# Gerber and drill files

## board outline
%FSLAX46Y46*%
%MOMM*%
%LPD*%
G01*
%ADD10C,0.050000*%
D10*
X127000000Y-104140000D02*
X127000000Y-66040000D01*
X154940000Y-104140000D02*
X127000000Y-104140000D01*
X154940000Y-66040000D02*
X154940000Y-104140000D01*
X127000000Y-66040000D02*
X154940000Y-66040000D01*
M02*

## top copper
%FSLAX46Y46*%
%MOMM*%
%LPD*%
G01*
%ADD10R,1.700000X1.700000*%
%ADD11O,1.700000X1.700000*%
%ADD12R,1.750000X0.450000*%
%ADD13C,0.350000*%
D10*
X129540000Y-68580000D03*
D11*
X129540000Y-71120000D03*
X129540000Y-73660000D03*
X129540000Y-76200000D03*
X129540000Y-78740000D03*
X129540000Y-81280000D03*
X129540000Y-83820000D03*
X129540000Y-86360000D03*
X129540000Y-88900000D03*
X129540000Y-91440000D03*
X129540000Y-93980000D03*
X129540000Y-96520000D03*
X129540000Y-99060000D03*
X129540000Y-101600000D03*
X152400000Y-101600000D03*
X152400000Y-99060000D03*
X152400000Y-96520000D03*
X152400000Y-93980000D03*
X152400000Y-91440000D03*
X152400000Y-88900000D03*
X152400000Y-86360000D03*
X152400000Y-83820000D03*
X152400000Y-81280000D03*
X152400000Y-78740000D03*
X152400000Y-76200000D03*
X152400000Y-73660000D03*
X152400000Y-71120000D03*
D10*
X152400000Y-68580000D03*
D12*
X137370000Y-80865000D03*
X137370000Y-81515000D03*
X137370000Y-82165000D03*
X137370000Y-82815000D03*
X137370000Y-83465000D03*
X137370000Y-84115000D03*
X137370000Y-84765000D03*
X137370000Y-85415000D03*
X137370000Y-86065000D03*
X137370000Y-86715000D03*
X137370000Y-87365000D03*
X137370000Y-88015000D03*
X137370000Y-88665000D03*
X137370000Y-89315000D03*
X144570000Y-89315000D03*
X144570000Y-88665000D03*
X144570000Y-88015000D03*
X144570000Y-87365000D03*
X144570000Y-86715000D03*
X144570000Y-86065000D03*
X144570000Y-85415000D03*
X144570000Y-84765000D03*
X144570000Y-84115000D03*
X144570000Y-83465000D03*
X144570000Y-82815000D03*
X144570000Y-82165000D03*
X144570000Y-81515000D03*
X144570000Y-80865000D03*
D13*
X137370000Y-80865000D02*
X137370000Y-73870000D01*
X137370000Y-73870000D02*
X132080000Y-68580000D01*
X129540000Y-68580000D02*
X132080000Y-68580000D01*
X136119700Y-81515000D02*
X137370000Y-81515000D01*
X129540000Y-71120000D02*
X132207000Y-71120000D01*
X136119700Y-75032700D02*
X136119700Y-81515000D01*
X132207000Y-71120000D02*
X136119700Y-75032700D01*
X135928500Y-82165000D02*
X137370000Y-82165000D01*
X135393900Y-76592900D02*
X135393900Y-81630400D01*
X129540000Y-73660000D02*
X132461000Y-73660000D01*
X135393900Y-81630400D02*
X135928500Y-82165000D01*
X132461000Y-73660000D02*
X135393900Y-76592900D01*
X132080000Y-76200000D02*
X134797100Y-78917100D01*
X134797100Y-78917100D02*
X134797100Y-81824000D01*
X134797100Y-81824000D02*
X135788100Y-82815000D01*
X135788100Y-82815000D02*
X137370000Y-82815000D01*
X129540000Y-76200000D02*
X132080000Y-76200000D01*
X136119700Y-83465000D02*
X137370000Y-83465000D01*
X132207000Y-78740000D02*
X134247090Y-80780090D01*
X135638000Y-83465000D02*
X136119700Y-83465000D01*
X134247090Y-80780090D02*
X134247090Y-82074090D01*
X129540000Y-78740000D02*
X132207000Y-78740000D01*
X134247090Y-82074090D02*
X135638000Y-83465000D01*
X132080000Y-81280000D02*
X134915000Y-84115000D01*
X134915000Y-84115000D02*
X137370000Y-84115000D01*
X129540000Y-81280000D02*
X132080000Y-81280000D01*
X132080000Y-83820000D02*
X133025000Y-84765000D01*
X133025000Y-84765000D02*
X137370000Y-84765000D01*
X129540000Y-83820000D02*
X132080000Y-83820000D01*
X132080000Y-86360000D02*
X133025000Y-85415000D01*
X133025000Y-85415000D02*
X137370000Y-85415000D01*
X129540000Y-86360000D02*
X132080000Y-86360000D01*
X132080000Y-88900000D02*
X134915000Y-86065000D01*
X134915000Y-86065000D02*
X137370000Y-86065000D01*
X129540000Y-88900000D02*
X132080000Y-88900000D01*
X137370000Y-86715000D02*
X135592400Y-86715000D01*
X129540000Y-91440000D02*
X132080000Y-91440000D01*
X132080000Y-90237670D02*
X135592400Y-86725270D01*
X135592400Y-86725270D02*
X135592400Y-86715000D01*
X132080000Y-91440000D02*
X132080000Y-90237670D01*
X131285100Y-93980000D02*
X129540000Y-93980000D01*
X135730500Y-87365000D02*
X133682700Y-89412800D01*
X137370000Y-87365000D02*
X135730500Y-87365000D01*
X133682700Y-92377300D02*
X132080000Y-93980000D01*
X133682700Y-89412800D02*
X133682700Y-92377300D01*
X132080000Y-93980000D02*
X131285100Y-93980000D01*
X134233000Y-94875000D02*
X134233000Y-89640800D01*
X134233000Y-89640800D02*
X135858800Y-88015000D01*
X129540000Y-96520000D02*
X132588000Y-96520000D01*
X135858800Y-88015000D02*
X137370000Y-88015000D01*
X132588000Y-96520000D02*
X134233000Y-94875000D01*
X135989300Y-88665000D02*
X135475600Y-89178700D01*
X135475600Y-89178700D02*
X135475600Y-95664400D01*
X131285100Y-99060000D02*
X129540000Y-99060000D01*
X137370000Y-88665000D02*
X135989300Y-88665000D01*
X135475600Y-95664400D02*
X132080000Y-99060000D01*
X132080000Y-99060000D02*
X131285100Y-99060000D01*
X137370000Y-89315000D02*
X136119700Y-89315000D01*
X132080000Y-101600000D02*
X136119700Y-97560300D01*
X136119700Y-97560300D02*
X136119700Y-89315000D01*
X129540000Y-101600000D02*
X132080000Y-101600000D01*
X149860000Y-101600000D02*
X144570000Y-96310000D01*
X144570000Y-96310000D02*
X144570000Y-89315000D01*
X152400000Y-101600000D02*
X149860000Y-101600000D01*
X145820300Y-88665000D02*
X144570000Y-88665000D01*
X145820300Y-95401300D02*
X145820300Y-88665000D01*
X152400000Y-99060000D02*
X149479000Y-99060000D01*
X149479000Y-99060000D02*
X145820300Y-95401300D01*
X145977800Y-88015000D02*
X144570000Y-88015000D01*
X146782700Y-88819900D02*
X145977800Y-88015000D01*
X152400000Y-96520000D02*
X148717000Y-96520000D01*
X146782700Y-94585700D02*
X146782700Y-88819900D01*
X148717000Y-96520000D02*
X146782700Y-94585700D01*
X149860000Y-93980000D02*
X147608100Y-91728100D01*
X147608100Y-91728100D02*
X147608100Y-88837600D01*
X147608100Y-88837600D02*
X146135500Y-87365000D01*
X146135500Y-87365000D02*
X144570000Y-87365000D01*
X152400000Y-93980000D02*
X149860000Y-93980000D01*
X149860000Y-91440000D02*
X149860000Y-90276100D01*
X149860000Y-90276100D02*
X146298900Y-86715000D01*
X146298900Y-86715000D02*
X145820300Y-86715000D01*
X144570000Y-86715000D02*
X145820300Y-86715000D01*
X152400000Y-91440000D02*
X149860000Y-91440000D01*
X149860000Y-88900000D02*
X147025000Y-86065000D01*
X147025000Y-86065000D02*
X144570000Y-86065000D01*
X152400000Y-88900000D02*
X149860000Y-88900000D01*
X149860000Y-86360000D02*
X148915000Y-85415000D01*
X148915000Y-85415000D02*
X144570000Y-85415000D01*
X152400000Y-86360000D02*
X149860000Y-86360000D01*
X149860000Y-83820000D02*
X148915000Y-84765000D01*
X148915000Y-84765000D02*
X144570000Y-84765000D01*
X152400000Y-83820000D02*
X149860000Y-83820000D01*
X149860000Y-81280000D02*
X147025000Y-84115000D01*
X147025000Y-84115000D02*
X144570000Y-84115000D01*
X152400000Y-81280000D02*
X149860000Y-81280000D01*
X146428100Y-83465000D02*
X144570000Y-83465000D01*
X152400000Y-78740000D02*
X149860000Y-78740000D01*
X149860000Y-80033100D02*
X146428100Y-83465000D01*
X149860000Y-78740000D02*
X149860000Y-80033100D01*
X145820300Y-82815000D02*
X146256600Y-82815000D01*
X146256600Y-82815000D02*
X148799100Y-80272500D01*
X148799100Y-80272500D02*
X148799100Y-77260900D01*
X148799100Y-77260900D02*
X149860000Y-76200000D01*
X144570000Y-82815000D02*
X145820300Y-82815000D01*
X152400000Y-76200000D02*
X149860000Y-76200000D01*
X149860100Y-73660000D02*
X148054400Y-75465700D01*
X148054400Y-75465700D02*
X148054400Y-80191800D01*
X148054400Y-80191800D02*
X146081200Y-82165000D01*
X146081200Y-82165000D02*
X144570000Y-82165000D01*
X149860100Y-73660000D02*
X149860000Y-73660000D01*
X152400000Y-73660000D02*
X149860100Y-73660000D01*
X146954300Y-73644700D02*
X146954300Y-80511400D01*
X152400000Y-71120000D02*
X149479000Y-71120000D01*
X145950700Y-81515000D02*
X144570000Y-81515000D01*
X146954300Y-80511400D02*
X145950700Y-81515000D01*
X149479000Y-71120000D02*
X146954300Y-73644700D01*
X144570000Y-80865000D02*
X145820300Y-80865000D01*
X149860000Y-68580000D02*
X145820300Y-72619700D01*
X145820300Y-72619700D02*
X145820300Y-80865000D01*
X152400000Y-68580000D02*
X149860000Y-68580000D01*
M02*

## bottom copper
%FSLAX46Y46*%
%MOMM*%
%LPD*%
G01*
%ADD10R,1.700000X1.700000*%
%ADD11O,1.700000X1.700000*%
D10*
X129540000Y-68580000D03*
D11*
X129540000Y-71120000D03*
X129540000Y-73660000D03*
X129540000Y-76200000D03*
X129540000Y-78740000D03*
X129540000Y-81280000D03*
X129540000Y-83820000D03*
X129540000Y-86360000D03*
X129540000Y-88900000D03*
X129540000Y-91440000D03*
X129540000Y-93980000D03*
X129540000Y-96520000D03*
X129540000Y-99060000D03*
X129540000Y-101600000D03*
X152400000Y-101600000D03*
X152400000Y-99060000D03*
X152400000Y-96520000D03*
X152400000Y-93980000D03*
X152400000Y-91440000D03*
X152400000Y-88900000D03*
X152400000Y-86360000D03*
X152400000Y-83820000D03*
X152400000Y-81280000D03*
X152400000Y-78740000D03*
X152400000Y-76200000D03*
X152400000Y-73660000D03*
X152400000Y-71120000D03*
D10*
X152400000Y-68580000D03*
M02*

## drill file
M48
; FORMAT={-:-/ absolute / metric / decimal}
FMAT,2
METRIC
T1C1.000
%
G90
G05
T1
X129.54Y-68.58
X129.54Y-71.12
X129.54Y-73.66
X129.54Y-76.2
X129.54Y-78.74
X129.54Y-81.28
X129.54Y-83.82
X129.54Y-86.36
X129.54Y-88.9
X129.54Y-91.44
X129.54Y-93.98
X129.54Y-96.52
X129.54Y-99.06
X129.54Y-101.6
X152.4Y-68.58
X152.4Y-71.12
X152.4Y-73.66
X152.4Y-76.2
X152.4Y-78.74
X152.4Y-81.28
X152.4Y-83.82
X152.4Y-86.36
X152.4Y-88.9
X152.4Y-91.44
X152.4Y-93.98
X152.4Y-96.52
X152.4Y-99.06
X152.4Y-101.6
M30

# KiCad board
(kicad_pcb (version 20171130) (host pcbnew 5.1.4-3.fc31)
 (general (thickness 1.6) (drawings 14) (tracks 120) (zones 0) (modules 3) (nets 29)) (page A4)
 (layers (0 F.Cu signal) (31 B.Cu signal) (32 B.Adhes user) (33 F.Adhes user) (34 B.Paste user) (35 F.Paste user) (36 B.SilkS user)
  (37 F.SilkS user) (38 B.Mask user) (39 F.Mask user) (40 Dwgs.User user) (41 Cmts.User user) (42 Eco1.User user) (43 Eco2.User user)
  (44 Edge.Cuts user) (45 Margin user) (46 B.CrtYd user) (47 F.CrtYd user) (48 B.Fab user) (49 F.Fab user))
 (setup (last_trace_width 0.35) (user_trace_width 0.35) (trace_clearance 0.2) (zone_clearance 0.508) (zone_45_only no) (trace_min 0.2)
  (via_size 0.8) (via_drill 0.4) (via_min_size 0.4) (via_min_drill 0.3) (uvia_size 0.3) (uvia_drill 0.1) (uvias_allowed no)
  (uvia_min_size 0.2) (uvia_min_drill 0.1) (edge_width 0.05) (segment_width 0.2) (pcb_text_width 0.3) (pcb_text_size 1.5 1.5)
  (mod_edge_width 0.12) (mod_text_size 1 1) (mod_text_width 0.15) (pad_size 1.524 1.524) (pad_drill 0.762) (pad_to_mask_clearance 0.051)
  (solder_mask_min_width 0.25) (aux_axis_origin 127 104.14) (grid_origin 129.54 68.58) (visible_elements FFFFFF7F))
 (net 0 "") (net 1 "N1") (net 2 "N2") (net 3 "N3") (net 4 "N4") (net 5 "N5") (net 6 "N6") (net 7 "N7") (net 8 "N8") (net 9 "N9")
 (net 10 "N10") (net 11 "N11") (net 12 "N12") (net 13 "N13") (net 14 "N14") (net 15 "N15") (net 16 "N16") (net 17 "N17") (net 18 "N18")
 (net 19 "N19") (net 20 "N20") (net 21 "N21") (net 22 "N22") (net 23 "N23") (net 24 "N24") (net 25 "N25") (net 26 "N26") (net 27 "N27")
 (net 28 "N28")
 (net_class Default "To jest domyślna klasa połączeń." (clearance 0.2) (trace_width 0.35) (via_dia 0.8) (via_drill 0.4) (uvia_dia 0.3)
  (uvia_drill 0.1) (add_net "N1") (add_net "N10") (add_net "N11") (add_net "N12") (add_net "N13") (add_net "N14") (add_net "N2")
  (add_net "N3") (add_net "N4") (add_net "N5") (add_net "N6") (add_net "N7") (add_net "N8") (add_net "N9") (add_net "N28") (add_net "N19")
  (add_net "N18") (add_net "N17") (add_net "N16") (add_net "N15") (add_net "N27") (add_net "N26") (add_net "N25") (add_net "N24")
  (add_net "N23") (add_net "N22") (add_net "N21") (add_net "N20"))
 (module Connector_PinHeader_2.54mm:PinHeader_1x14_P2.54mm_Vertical (layer B.Cu) (at 129.54 68.58 180)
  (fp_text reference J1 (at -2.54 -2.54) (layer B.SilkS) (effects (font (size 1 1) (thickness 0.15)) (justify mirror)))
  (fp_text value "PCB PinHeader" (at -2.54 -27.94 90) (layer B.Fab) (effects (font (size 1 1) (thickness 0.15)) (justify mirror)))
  (pad 1 thru_hole rect (at 0 0 180) (size 1.7 1.7) (drill 1) (layers *.Cu *.Mask) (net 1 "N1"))
  (pad 2 thru_hole oval (at 0 -2.54 180) (size 1.7 1.7) (drill 1) (layers *.Cu *.Mask) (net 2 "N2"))
  (pad 3 thru_hole oval (at 0 -5.08 180) (size 1.7 1.7) (drill 1) (layers *.Cu *.Mask) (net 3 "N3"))
  (pad 4 thru_hole oval (at 0 -7.62 180) (size 1.7 1.7) (drill 1) (layers *.Cu *.Mask) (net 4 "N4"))
  (pad 5 thru_hole oval (at 0 -10.16 180) (size 1.7 1.7) (drill 1) (layers *.Cu *.Mask) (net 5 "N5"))
  (pad 6 thru_hole oval (at 0 -12.7 180) (size 1.7 1.7) (drill 1) (layers *.Cu *.Mask) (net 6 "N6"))
  (pad 7 thru_hole oval (at 0 -15.24 180) (size 1.7 1.7) (drill 1) (layers *.Cu *.Mask) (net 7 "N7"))
  (pad 8 thru_hole oval (at 0 -17.78 180) (size 1.7 1.7) (drill 1) (layers *.Cu *.Mask) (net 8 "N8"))
  (pad 9 thru_hole oval (at 0 -20.32 180) (size 1.7 1.7) (drill 1) (layers *.Cu *.Mask) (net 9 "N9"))
  (pad 10 thru_hole oval (at 0 -22.86 180) (size 1.7 1.7) (drill 1) (layers *.Cu *.Mask) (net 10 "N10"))
  (pad 11 thru_hole oval (at 0 -25.4 180) (size 1.7 1.7) (drill 1) (layers *.Cu *.Mask) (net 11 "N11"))
  (pad 12 thru_hole oval (at 0 -27.94 180) (size 1.7 1.7) (drill 1) (layers *.Cu *.Mask) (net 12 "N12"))
  (pad 13 thru_hole oval (at 0 -30.48 180) (size 1.7 1.7) (drill 1) (layers *.Cu *.Mask) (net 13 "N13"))
  (pad 14 thru_hole oval (at 0 -33.02 180) (size 1.7 1.7) (drill 1) (layers *.Cu *.Mask) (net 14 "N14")))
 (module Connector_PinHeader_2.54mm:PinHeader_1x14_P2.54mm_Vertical (layer B.Cu) (at 152.4 68.58 180)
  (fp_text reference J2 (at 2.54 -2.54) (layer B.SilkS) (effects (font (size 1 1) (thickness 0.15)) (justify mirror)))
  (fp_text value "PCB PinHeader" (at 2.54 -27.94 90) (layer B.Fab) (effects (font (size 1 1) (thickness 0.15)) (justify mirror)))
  (pad 14 thru_hole oval (at 0 -33.02 180) (size 1.7 1.7) (drill 1) (layers *.Cu *.Mask) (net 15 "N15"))
  (pad 13 thru_hole oval (at 0 -30.48 180) (size 1.7 1.7) (drill 1) (layers *.Cu *.Mask) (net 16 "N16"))
  (pad 12 thru_hole oval (at 0 -27.94 180) (size 1.7 1.7) (drill 1) (layers *.Cu *.Mask) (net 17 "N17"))
  (pad 11 thru_hole oval (at 0 -25.4 180) (size 1.7 1.7) (drill 1) (layers *.Cu *.Mask) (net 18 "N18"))
  (pad 10 thru_hole oval (at 0 -22.86 180) (size 1.7 1.7) (drill 1) (layers *.Cu *.Mask) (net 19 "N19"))
  (pad 9 thru_hole oval (at 0 -20.32 180) (size 1.7 1.7) (drill 1) (layers *.Cu *.Mask) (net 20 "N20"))
  (pad 8 thru_hole oval (at 0 -17.78 180) (size 1.7 1.7) (drill 1) (layers *.Cu *.Mask) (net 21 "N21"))
  (pad 7 thru_hole oval (at 0 -15.24 180) (size 1.7 1.7) (drill 1) (layers *.Cu *.Mask) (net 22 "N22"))
  (pad 6 thru_hole oval (at 0 -12.7 180) (size 1.7 1.7) (drill 1) (layers *.Cu *.Mask) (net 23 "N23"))
  (pad 5 thru_hole oval (at 0 -10.16 180) (size 1.7 1.7) (drill 1) (layers *.Cu *.Mask) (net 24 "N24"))
  (pad 4 thru_hole oval (at 0 -7.62 180) (size 1.7 1.7) (drill 1) (layers *.Cu *.Mask) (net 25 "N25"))
  (pad 3 thru_hole oval (at 0 -5.08 180) (size 1.7 1.7) (drill 1) (layers *.Cu *.Mask) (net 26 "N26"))
  (pad 2 thru_hole oval (at 0 -2.54 180) (size 1.7 1.7) (drill 1) (layers *.Cu *.Mask) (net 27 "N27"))
  (pad 1 thru_hole rect (at 0 0 180) (size 1.7 1.7) (drill 1) (layers *.Cu *.Mask) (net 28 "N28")))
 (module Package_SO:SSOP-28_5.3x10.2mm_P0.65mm (layer F.Cu) (at 140.97 85.09)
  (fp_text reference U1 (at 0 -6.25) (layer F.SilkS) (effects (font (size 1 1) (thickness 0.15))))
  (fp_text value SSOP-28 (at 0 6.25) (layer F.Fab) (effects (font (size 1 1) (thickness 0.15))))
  (pad 1 smd rect (at -3.6 -4.225) (size 1.75 0.45) (layers F.Cu F.Paste F.Mask) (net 1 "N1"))
  (pad 2 smd rect (at -3.6 -3.575) (size 1.75 0.45) (layers F.Cu F.Paste F.Mask) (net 2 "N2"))
  (pad 3 smd rect (at -3.6 -2.925) (size 1.75 0.45) (layers F.Cu F.Paste F.Mask) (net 3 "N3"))
  (pad 4 smd rect (at -3.6 -2.275) (size 1.75 0.45) (layers F.Cu F.Paste F.Mask) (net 4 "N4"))
  (pad 5 smd rect (at -3.6 -1.625) (size 1.75 0.45) (layers F.Cu F.Paste F.Mask) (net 5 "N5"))
  (pad 6 smd rect (at -3.6 -0.975) (size 1.75 0.45) (layers F.Cu F.Paste F.Mask) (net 6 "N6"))
  (pad 7 smd rect (at -3.6 -0.325) (size 1.75 0.45) (layers F.Cu F.Paste F.Mask) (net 7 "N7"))
  (pad 8 smd rect (at -3.6 0.325) (size 1.75 0.45) (layers F.Cu F.Paste F.Mask) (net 8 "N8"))
  (pad 9 smd rect (at -3.6 0.975) (size 1.75 0.45) (layers F.Cu F.Paste F.Mask) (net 9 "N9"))
  (pad 10 smd rect (at -3.6 1.625) (size 1.75 0.45) (layers F.Cu F.Paste F.Mask) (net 10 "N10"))
  (pad 11 smd rect (at -3.6 2.275) (size 1.75 0.45) (layers F.Cu F.Paste F.Mask) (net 11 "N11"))
  (pad 12 smd rect (at -3.6 2.925) (size 1.75 0.45) (layers F.Cu F.Paste F.Mask) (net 12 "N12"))
  (pad 13 smd rect (at -3.6 3.575) (size 1.75 0.45) (layers F.Cu F.Paste F.Mask) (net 13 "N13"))
  (pad 14 smd rect (at -3.6 4.225) (size 1.75 0.45) (layers F.Cu F.Paste F.Mask) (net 14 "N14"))
  (pad 15 smd rect (at 3.6 4.225) (size 1.75 0.45) (layers F.Cu F.Paste F.Mask) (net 15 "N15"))
  (pad 16 smd rect (at 3.6 3.575) (size 1.75 0.45) (layers F.Cu F.Paste F.Mask) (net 16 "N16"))
  (pad 17 smd rect (at 3.6 2.925) (size 1.75 0.45) (layers F.Cu F.Paste F.Mask) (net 17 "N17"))
  (pad 18 smd rect (at 3.6 2.275) (size 1.75 0.45) (layers F.Cu F.Paste F.Mask) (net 18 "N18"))
  (pad 19 smd rect (at 3.6 1.625) (size 1.75 0.45) (layers F.Cu F.Paste F.Mask) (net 19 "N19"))
  (pad 20 smd rect (at 3.6 0.975) (size 1.75 0.45) (layers F.Cu F.Paste F.Mask) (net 20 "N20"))
  (pad 21 smd rect (at 3.6 0.325) (size 1.75 0.45) (layers F.Cu F.Paste F.Mask) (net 21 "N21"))
  (pad 22 smd rect (at 3.6 -0.325) (size 1.75 0.45) (layers F.Cu F.Paste F.Mask) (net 22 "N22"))
  (pad 23 smd rect (at 3.6 -0.975) (size 1.75 0.45) (layers F.Cu F.Paste F.Mask) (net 23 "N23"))
  (pad 24 smd rect (at 3.6 -1.625) (size 1.75 0.45) (layers F.Cu F.Paste F.Mask) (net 24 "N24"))
  (pad 25 smd rect (at 3.6 -2.275) (size 1.75 0.45) (layers F.Cu F.Paste F.Mask) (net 25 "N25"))
  (pad 26 smd rect (at 3.6 -2.925) (size 1.75 0.45) (layers F.Cu F.Paste F.Mask) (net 26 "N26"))
  (pad 27 smd rect (at 3.6 -3.575) (size 1.75 0.45) (layers F.Cu F.Paste F.Mask) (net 27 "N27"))
  (pad 28 smd rect (at 3.6 -4.225) (size 1.75 0.45) (layers F.Cu F.Paste F.Mask) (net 28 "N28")))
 (gr_line (start 127 104.14) (end 127 66.04) (layer Edge.Cuts) (width 0.05))
 (gr_line (start 154.94 104.14) (end 127 104.14) (layer Edge.Cuts) (width 0.05))
 (gr_line (start 154.94 66.04) (end 154.94 104.14) (layer Edge.Cuts) (width 0.05))
 (gr_line (start 127 66.04) (end 154.94 66.04) (layer Edge.Cuts) (width 0.05))
 (segment (start 137.37 80.865) (end 137.37 73.87) (width 0.35) (layer F.Cu) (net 1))
 (segment (start 137.37 73.87) (end 132.08 68.58) (width 0.35) (layer F.Cu) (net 1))
 (segment (start 129.54 68.58) (end 132.08 68.58) (width 0.35) (layer F.Cu) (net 1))
 (segment (start 136.1197 81.515) (end 137.37 81.515) (width 0.35) (layer F.Cu) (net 2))
 (segment (start 129.54 71.12) (end 132.207 71.12) (width 0.35) (layer F.Cu) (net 2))
 (segment (start 136.1197 75.0327) (end 136.1197 81.515) (width 0.35) (layer F.Cu) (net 2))
 (segment (start 132.207 71.12) (end 136.1197 75.0327) (width 0.35) (layer F.Cu) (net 2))
 (segment (start 135.9285 82.165) (end 137.37 82.165) (width 0.35) (layer F.Cu) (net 3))
 (segment (start 135.3939 76.5929) (end 135.3939 81.6304) (width 0.35) (layer F.Cu) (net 3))
 (segment (start 129.54 73.66) (end 132.461 73.66) (width 0.35) (layer F.Cu) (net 3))
 (segment (start 135.3939 81.6304) (end 135.9285 82.165) (width 0.35) (layer F.Cu) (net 3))
 (segment (start 132.461 73.66) (end 135.3939 76.5929) (width 0.35) (layer F.Cu) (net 3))
 (segment (start 132.08 76.2) (end 134.7971 78.9171) (width 0.35) (layer F.Cu) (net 4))
 (segment (start 134.7971 78.9171) (end 134.7971 81.824) (width 0.35) (layer F.Cu) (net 4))
 (segment (start 134.7971 81.824) (end 135.7881 82.815) (width 0.35) (layer F.Cu) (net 4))
 (segment (start 135.7881 82.815) (end 137.37 82.815) (width 0.35) (layer F.Cu) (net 4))
 (segment (start 129.54 76.2) (end 132.08 76.2) (width 0.35) (layer F.Cu) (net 4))
 (segment (start 136.1197 83.465) (end 137.37 83.465) (width 0.35) (layer F.Cu) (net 5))
 (segment (start 132.207 78.74) (end 134.24709 80.78009) (width 0.35) (layer F.Cu) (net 5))
 (segment (start 135.638 83.465) (end 136.1197 83.465) (width 0.35) (layer F.Cu) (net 5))
 (segment (start 134.24709 80.78009) (end 134.24709 82.07409) (width 0.35) (layer F.Cu) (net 5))
 (segment (start 129.54 78.74) (end 132.207 78.74) (width 0.35) (layer F.Cu) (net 5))
 (segment (start 134.24709 82.07409) (end 135.638 83.465) (width 0.35) (layer F.Cu) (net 5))
 (segment (start 132.08 81.28) (end 134.915 84.115) (width 0.35) (layer F.Cu) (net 6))
 (segment (start 134.915 84.115) (end 137.37 84.115) (width 0.35) (layer F.Cu) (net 6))
 (segment (start 129.54 81.28) (end 132.08 81.28) (width 0.35) (layer F.Cu) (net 6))
 (segment (start 132.08 83.82) (end 133.025 84.765) (width 0.35) (layer F.Cu) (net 7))
 (segment (start 133.025 84.765) (end 137.37 84.765) (width 0.35) (layer F.Cu) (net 7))
 (segment (start 129.54 83.82) (end 132.08 83.82) (width 0.35) (layer F.Cu) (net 7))
 (segment (start 132.08 86.36) (end 133.025 85.415) (width 0.35) (layer F.Cu) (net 8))
 (segment (start 133.025 85.415) (end 137.37 85.415) (width 0.35) (layer F.Cu) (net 8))
 (segment (start 129.54 86.36) (end 132.08 86.36) (width 0.35) (layer F.Cu) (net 8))
 (segment (start 132.08 88.9) (end 134.915 86.065) (width 0.35) (layer F.Cu) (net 9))
 (segment (start 134.915 86.065) (end 137.37 86.065) (width 0.35) (layer F.Cu) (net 9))
 (segment (start 129.54 88.9) (end 132.08 88.9) (width 0.35) (layer F.Cu) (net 9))
 (segment (start 137.37 86.715) (end 135.5924 86.715) (width 0.35) (layer F.Cu) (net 10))
 (segment (start 129.54 91.44) (end 132.08 91.44) (width 0.35) (layer F.Cu) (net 10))
 (segment (start 132.08 90.23767) (end 135.5924 86.72527) (width 0.35) (layer F.Cu) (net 10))
 (segment (start 135.5924 86.72527) (end 135.5924 86.715) (width 0.35) (layer F.Cu) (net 10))
 (segment (start 132.08 91.44) (end 132.08 90.23767) (width 0.35) (layer F.Cu) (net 10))
 (segment (start 131.2851 93.98) (end 129.54 93.98) (width 0.35) (layer F.Cu) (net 11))
 (segment (start 135.7305 87.365) (end 133.6827 89.4128) (width 0.35) (layer F.Cu) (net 11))
 (segment (start 137.37 87.365) (end 135.7305 87.365) (width 0.35) (layer F.Cu) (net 11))
 (segment (start 133.6827 92.3773) (end 132.08 93.98) (width 0.35) (layer F.Cu) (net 11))
 (segment (start 133.6827 89.4128) (end 133.6827 92.3773) (width 0.35) (layer F.Cu) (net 11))
 (segment (start 132.08 93.98) (end 131.2851 93.98) (width 0.35) (layer F.Cu) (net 11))
 (segment (start 134.233 94.875) (end 134.233 89.6408) (width 0.35) (layer F.Cu) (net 12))
 (segment (start 134.233 89.6408) (end 135.8588 88.015) (width 0.35) (layer F.Cu) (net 12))
 (segment (start 129.54 96.52) (end 132.588 96.52) (width 0.35) (layer F.Cu) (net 12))
 (segment (start 135.8588 88.015) (end 137.37 88.015) (width 0.35) (layer F.Cu) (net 12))
 (segment (start 132.588 96.52) (end 134.233 94.875) (width 0.35) (layer F.Cu) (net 12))
 (segment (start 135.9893 88.665) (end 135.4756 89.1787) (width 0.35) (layer F.Cu) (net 13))
 (segment (start 135.4756 89.1787) (end 135.4756 95.6644) (width 0.35) (layer F.Cu) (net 13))
 (segment (start 131.2851 99.06) (end 129.54 99.06) (width 0.35) (layer F.Cu) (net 13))
 (segment (start 137.37 88.665) (end 135.9893 88.665) (width 0.35) (layer F.Cu) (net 13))
 (segment (start 135.4756 95.6644) (end 132.08 99.06) (width 0.35) (layer F.Cu) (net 13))
 (segment (start 132.08 99.06) (end 131.2851 99.06) (width 0.35) (layer F.Cu) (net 13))
 (segment (start 137.37 89.315) (end 136.1197 89.315) (width 0.35) (layer F.Cu) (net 14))
 (segment (start 132.08 101.6) (end 136.1197 97.5603) (width 0.35) (layer F.Cu) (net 14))
 (segment (start 136.1197 97.5603) (end 136.1197 89.315) (width 0.35) (layer F.Cu) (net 14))
 (segment (start 129.54 101.6) (end 132.08 101.6) (width 0.35) (layer F.Cu) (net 14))
 (segment (start 149.86 101.6) (end 144.57 96.31) (width 0.35) (layer F.Cu) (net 15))
 (segment (start 144.57 96.31) (end 144.57 89.315) (width 0.35) (layer F.Cu) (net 15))
 (segment (start 152.4 101.6) (end 149.86 101.6) (width 0.35) (layer F.Cu) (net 15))
 (segment (start 145.8203 88.665) (end 144.57 88.665) (width 0.35) (layer F.Cu) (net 16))
 (segment (start 145.8203 95.4013) (end 145.8203 88.665) (width 0.35) (layer F.Cu) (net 16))
 (segment (start 152.4 99.06) (end 149.479 99.06) (width 0.35) (layer F.Cu) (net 16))
 (segment (start 149.479 99.06) (end 145.8203 95.4013) (width 0.35) (layer F.Cu) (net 16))
 (segment (start 145.9778 88.015) (end 144.57 88.015) (width 0.35) (layer F.Cu) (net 17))
 (segment (start 146.7827 88.8199) (end 145.9778 88.015) (width 0.35) (layer F.Cu) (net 17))
 (segment (start 152.4 96.52) (end 148.717 96.52) (width 0.35) (layer F.Cu) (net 17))
 (segment (start 146.7827 94.5857) (end 146.7827 88.8199) (width 0.35) (layer F.Cu) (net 17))
 (segment (start 148.717 96.52) (end 146.7827 94.5857) (width 0.35) (layer F.Cu) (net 17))
 (segment (start 149.86 93.98) (end 147.6081 91.7281) (width 0.35) (layer F.Cu) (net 18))
 (segment (start 147.6081 91.7281) (end 147.6081 88.8376) (width 0.35) (layer F.Cu) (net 18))
 (segment (start 147.6081 88.8376) (end 146.1355 87.365) (width 0.35) (layer F.Cu) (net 18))
 (segment (start 146.1355 87.365) (end 144.57 87.365) (width 0.35) (layer F.Cu) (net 18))
 (segment (start 152.4 93.98) (end 149.86 93.98) (width 0.35) (layer F.Cu) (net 18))
 (segment (start 149.86 91.44) (end 149.86 90.2761) (width 0.35) (layer F.Cu) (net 19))
 (segment (start 149.86 90.2761) (end 146.2989 86.715) (width 0.35) (layer F.Cu) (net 19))
 (segment (start 146.2989 86.715) (end 145.8203 86.715) (width 0.35) (layer F.Cu) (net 19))
 (segment (start 144.57 86.715) (end 145.8203 86.715) (width 0.35) (layer F.Cu) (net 19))
 (segment (start 152.4 91.44) (end 149.86 91.44) (width 0.35) (layer F.Cu) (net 19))
 (segment (start 149.86 88.9) (end 147.025 86.065) (width 0.35) (layer F.Cu) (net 20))
 (segment (start 147.025 86.065) (end 144.57 86.065) (width 0.35) (layer F.Cu) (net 20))
 (segment (start 152.4 88.9) (end 149.86 88.9) (width 0.35) (layer F.Cu) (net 20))
 (segment (start 149.86 86.36) (end 148.915 85.415) (width 0.35) (layer F.Cu) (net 21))
 (segment (start 148.915 85.415) (end 144.57 85.415) (width 0.35) (layer F.Cu) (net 21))
 (segment (start 152.4 86.36) (end 149.86 86.36) (width 0.35) (layer F.Cu) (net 21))
 (segment (start 149.86 83.82) (end 148.915 84.765) (width 0.35) (layer F.Cu) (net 22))
 (segment (start 148.915 84.765) (end 144.57 84.765) (width 0.35) (layer F.Cu) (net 22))
 (segment (start 152.4 83.82) (end 149.86 83.82) (width 0.35) (layer F.Cu) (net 22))
 (segment (start 149.86 81.28) (end 147.025 84.115) (width 0.35) (layer F.Cu) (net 23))
 (segment (start 147.025 84.115) (end 144.57 84.115) (width 0.35) (layer F.Cu) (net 23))
 (segment (start 152.4 81.28) (end 149.86 81.28) (width 0.35) (layer F.Cu) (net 23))
 (segment (start 146.4281 83.465) (end 144.57 83.465) (width 0.35) (layer F.Cu) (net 24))
 (segment (start 152.4 78.74) (end 149.86 78.74) (width 0.35) (layer F.Cu) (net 24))
 (segment (start 149.86 80.0331) (end 146.4281 83.465) (width 0.35) (layer F.Cu) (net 24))
 (segment (start 149.86 78.74) (end 149.86 80.0331) (width 0.35) (layer F.Cu) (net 24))
 (segment (start 145.8203 82.815) (end 146.2566 82.815) (width 0.35) (layer F.Cu) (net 25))
 (segment (start 146.2566 82.815) (end 148.7991 80.2725) (width 0.35) (layer F.Cu) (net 25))
 (segment (start 148.7991 80.2725) (end 148.7991 77.2609) (width 0.35) (layer F.Cu) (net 25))
 (segment (start 148.7991 77.2609) (end 149.86 76.2) (width 0.35) (layer F.Cu) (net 25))
 (segment (start 144.57 82.815) (end 145.8203 82.815) (width 0.35) (layer F.Cu) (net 25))
 (segment (start 152.4 76.2) (end 149.86 76.2) (width 0.35) (layer F.Cu) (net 25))
 (segment (start 149.8601 73.66) (end 148.0544 75.4657) (width 0.35) (layer F.Cu) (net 26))
 (segment (start 148.0544 75.4657) (end 148.0544 80.1918) (width 0.35) (layer F.Cu) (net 26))
 (segment (start 148.0544 80.1918) (end 146.0812 82.165) (width 0.35) (layer F.Cu) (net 26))
 (segment (start 146.0812 82.165) (end 144.57 82.165) (width 0.35) (layer F.Cu) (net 26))
 (segment (start 149.8601 73.66) (end 149.86 73.66) (width 0.35) (layer F.Cu) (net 26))
 (segment (start 152.4 73.66) (end 149.8601 73.66) (width 0.35) (layer F.Cu) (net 26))
 (segment (start 146.9543 73.6447) (end 146.9543 80.5114) (width 0.35) (layer F.Cu) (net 27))
 (segment (start 152.4 71.12) (end 149.479 71.12) (width 0.35) (layer F.Cu) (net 27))
 (segment (start 145.9507 81.515) (end 144.57 81.515) (width 0.35) (layer F.Cu) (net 27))
 (segment (start 146.9543 80.5114) (end 145.9507 81.515) (width 0.35) (layer F.Cu) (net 27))
 (segment (start 149.479 71.12) (end 146.9543 73.6447) (width 0.35) (layer F.Cu) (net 27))
 (segment (start 144.57 80.865) (end 145.8203 80.865) (width 0.35) (layer F.Cu) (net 28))
 (segment (start 149.86 68.58) (end 145.8203 72.6197) (width 0.35) (layer F.Cu) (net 28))
 (segment (start 145.8203 72.6197) (end 145.8203 80.865) (width 0.35) (layer F.Cu) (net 28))
 (segment (start 152.4 68.58) (end 149.86 68.58) (width 0.35) (layer F.Cu) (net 28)))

